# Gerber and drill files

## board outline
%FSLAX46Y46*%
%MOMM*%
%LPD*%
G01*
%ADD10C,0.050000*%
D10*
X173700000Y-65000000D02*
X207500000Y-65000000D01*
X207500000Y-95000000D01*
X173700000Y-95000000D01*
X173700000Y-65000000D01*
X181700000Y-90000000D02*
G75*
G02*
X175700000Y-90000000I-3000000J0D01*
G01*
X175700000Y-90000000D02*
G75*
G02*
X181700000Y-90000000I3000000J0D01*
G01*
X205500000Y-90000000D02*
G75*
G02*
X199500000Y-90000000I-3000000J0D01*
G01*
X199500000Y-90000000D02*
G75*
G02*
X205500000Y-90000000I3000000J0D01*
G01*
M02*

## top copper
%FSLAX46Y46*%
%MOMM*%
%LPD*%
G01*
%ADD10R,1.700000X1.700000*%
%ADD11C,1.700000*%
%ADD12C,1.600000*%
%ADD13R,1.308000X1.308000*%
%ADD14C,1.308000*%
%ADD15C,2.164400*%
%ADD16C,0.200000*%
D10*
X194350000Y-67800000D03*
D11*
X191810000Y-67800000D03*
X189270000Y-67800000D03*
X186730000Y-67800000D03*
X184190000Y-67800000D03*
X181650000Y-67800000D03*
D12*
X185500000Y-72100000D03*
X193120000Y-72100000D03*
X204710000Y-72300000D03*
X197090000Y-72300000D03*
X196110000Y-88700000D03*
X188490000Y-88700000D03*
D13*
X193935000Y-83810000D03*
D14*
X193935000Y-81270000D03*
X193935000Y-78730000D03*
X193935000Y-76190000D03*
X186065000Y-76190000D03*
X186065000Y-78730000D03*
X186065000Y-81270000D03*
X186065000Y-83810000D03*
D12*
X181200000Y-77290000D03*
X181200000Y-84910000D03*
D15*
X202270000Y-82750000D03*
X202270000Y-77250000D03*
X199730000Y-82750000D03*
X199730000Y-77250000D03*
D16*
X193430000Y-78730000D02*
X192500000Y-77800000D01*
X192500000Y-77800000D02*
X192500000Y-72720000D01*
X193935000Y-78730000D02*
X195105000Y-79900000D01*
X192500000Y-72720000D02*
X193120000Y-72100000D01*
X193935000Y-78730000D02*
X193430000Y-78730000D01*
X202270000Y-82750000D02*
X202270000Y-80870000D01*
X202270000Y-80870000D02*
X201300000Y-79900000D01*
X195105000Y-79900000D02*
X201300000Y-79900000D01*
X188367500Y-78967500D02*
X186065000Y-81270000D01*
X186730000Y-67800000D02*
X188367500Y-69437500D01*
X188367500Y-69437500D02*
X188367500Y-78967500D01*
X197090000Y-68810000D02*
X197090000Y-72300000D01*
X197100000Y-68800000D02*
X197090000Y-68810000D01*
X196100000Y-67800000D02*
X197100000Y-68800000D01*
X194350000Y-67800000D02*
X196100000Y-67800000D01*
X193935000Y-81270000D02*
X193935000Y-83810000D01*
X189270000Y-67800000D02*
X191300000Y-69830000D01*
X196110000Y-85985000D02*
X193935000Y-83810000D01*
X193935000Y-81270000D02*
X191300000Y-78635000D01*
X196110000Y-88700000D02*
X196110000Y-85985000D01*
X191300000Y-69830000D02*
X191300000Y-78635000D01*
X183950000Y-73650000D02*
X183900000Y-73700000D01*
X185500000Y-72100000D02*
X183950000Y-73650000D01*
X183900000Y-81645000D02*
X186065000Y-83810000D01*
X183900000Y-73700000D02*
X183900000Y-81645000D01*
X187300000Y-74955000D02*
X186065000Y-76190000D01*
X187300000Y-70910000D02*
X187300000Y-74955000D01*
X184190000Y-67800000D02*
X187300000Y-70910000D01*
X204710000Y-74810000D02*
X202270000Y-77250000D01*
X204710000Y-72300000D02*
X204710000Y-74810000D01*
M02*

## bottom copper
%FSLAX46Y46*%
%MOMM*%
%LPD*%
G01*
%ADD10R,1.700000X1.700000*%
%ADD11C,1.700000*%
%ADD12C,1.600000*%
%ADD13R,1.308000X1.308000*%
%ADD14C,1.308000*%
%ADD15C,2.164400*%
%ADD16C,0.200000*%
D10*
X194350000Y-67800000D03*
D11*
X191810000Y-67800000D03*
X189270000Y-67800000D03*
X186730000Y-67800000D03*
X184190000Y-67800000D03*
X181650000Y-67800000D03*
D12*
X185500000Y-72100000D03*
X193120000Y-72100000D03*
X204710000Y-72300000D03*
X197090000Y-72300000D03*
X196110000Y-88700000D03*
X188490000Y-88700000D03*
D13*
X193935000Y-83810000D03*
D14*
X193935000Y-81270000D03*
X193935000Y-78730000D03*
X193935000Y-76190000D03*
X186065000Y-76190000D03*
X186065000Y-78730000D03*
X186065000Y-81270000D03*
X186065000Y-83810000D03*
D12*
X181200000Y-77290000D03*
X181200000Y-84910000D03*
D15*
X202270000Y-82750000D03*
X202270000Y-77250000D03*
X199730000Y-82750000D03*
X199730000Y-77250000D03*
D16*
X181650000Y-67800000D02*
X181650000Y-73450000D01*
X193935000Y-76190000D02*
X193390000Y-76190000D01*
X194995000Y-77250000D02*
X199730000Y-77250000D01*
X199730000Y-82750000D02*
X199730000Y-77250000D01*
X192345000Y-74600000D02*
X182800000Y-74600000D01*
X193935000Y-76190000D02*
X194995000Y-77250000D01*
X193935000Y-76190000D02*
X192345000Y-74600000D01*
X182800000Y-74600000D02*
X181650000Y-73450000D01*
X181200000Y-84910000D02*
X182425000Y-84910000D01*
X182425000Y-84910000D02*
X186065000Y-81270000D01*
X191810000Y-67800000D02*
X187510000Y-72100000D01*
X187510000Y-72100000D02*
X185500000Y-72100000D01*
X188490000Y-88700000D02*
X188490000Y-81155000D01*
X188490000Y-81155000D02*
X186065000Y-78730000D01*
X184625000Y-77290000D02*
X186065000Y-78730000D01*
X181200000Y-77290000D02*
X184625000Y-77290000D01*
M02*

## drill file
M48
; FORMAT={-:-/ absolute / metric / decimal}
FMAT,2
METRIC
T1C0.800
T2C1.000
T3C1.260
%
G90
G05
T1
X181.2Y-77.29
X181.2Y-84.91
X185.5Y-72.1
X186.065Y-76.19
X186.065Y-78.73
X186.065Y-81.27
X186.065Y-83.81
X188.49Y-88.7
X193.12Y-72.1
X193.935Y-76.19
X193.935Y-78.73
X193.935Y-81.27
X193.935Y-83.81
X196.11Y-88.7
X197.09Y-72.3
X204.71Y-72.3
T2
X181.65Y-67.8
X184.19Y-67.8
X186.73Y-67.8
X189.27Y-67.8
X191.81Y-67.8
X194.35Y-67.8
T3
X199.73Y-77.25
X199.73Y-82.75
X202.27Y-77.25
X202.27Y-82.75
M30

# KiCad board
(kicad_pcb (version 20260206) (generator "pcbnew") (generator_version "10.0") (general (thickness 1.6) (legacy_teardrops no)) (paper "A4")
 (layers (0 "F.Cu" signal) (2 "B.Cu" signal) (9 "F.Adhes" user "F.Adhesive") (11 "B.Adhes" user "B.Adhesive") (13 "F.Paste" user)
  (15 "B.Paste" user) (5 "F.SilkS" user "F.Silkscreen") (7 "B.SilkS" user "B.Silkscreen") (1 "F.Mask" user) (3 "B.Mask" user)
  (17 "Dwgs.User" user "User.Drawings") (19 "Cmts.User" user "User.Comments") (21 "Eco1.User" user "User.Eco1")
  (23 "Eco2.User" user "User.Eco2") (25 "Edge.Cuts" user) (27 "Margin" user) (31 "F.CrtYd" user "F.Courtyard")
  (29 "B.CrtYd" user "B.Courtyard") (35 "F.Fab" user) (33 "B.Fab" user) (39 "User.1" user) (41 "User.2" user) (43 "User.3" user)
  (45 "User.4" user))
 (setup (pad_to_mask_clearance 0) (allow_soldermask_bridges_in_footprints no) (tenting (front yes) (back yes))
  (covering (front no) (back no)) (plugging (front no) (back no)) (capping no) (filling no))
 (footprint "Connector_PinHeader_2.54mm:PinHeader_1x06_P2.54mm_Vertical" (layer "F.Cu") (at 194.35 67.8 -90)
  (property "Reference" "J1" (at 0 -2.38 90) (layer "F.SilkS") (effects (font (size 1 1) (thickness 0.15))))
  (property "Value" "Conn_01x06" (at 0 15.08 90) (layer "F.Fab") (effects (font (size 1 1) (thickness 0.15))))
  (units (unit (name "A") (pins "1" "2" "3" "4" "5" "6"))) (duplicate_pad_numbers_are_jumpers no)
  (pad "1" thru_hole rect (at 0 0 270) (size 1.7 1.7) (drill 1) (layers "*.Cu" "*.Mask") (remove_unused_layers no) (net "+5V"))
  (pad "2" thru_hole circle (at 0 2.54 270) (size 1.7 1.7) (drill 1) (layers "*.Cu" "*.Mask") (remove_unused_layers no) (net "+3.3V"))
  (pad "3" thru_hole circle (at 0 5.08 270) (size 1.7 1.7) (drill 1) (layers "*.Cu" "*.Mask") (remove_unused_layers no) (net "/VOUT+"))
  (pad "4" thru_hole circle (at 0 7.62 270) (size 1.7 1.7) (drill 1) (layers "*.Cu" "*.Mask") (remove_unused_layers no) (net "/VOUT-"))
  (pad "5" thru_hole circle (at 0 10.16 270) (size 1.7 1.7) (drill 1) (layers "*.Cu" "*.Mask") (remove_unused_layers no) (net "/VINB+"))
  (pad "6" thru_hole circle (at 0 12.7 270) (size 1.7 1.7) (drill 1) (layers "*.Cu" "*.Mask") (remove_unused_layers no) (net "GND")))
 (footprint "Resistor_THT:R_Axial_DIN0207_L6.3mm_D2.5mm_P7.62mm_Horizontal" (layer "F.Cu") (at 185.5 72.1)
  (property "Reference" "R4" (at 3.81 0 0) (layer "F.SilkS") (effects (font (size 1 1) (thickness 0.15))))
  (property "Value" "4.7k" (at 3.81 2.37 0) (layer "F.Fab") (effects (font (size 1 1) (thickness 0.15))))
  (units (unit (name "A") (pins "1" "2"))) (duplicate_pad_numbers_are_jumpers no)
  (pad "1" thru_hole circle (at 0 0) (size 1.6 1.6) (drill 0.8) (layers "*.Cu" "*.Mask") (remove_unused_layers no) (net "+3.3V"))
  (pad "2" thru_hole circle (at 7.62 0) (size 1.6 1.6) (drill 0.8) (layers "*.Cu" "*.Mask") (remove_unused_layers no) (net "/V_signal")))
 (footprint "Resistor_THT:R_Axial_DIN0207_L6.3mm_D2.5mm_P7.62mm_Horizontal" (layer "F.Cu") (at 204.71 72.3 180)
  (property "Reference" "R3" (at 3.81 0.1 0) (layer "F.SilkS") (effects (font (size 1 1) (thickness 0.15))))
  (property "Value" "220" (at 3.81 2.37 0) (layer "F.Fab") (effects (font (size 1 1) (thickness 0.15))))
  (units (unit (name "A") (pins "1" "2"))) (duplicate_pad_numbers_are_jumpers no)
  (pad "1" thru_hole circle (at 0 0 180) (size 1.6 1.6) (drill 0.8) (layers "*.Cu" "*.Mask") (remove_unused_layers no) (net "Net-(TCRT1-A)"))
  (pad "2" thru_hole circle (at 7.62 0 180) (size 1.6 1.6) (drill 0.8) (layers "*.Cu" "*.Mask") (remove_unused_layers no) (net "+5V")))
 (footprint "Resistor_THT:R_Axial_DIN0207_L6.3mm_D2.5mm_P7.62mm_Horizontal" (layer "F.Cu") (at 196.11 88.7 180)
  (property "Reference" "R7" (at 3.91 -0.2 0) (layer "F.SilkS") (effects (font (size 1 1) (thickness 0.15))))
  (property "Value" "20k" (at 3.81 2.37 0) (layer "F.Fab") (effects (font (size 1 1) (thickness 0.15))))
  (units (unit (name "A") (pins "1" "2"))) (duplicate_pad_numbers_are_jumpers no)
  (pad "1" thru_hole circle (at 0 0 180) (size 1.6 1.6) (drill 0.8) (layers "*.Cu" "*.Mask") (remove_unused_layers no) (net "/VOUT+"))
  (pad "2" thru_hole circle (at 7.62 0 180) (size 1.6 1.6) (drill 0.8) (layers "*.Cu" "*.Mask") (remove_unused_layers no) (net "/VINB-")))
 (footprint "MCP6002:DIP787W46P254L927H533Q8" (layer "F.Cu") (at 190 80 180)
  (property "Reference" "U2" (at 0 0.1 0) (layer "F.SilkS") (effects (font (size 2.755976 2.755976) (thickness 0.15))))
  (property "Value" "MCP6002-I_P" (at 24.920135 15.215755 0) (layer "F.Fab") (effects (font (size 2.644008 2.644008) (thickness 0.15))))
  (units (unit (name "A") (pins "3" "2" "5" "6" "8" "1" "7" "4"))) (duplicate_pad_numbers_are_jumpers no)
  (pad "1" thru_hole rect (at -3.935 -3.81 180) (size 1.308 1.308) (drill 0.8) (layers "*.Cu" "*.Mask") (remove_unused_layers no)
   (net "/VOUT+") (solder_mask_margin 0.102))
  (pad "2" thru_hole circle (at -3.935 -1.27 180) (size 1.308 1.308) (drill 0.8) (layers "*.Cu" "*.Mask") (remove_unused_layers no)
   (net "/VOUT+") (solder_mask_margin 0.102))
  (pad "3" thru_hole circle (at -3.935 1.27 180) (size 1.308 1.308) (drill 0.8) (layers "*.Cu" "*.Mask") (remove_unused_layers no)
   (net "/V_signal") (solder_mask_margin 0.102))
  (pad "4" thru_hole circle (at -3.935 3.81 180) (size 1.308 1.308) (drill 0.8) (layers "*.Cu" "*.Mask") (remove_unused_layers no)
   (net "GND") (solder_mask_margin 0.102))
  (pad "5" thru_hole circle (at 3.935 3.81 180) (size 1.308 1.308) (drill 0.8) (layers "*.Cu" "*.Mask") (remove_unused_layers no)
   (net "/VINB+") (solder_mask_margin 0.102))
  (pad "6" thru_hole circle (at 3.935 1.27 180) (size 1.308 1.308) (drill 0.8) (layers "*.Cu" "*.Mask") (remove_unused_layers no)
   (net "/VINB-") (solder_mask_margin 0.102))
  (pad "7" thru_hole circle (at 3.935 -1.27 180) (size 1.308 1.308) (drill 0.8) (layers "*.Cu" "*.Mask") (remove_unused_layers no)
   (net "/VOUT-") (solder_mask_margin 0.102))
  (pad "8" thru_hole circle (at 3.935 -3.81 180) (size 1.308 1.308) (drill 0.8) (layers "*.Cu" "*.Mask") (remove_unused_layers no)
   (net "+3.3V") (solder_mask_margin 0.102)))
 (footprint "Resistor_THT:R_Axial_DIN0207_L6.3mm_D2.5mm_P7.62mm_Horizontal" (layer "F.Cu") (at 181.2 77.29 -90)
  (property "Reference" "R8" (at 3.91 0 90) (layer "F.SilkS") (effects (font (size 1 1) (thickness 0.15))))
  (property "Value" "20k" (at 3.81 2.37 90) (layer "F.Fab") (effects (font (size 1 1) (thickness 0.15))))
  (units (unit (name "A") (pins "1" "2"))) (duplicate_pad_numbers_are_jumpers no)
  (pad "1" thru_hole circle (at 0 0 270) (size 1.6 1.6) (drill 0.8) (layers "*.Cu" "*.Mask") (remove_unused_layers no) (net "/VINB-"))
  (pad "2" thru_hole circle (at 7.62 0 270) (size 1.6 1.6) (drill 0.8) (layers "*.Cu" "*.Mask") (remove_unused_layers no) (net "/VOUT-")))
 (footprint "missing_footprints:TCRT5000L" (layer "B.Cu") (at 201 80 90)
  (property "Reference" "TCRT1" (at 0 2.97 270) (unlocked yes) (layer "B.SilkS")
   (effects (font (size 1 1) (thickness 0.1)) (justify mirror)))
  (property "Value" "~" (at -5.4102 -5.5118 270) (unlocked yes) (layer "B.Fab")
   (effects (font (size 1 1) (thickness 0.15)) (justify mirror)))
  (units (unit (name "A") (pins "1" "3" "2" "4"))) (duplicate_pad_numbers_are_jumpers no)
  (pad "1" thru_hole circle (at -2.75 1.27 90) (size 2.1644 2.1644) (drill 1.26) (layers "*.Cu" "*.Mask") (remove_unused_layers no)
   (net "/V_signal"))
  (pad "2" thru_hole circle (at 2.75 1.27 90) (size 2.1644 2.1644) (drill 1.26) (layers "*.Cu" "*.Mask") (remove_unused_layers no)
   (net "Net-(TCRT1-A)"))
  (pad "3" thru_hole circle (at -2.75 -1.27 90) (size 2.1644 2.1644) (drill 1.26) (layers "*.Cu" "*.Mask") (remove_unused_layers no)
   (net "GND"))
  (pad "4" thru_hole circle (at 2.75 -1.27 90) (size 2.1644 2.1644) (drill 1.26) (layers "*.Cu" "*.Mask") (remove_unused_layers no)
   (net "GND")))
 (gr_rect (start 173.7 65) (end 207.5 95) (stroke (width 0.05) (type solid)) (fill no) (layer "Edge.Cuts"))
 (gr_circle (center 178.7 90) (end 181.7 90) (stroke (width 0.05) (type solid)) (fill no) (layer "Edge.Cuts"))
 (gr_circle (center 202.5 90) (end 205.5 90) (stroke (width 0.05) (type solid)) (fill no) (layer "Edge.Cuts"))
 (segment (start 181.65 67.8) (end 181.65 73.45) (width 0.2) (layer "B.Cu") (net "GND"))
 (segment (start 193.935 76.19) (end 193.39 76.19) (width 0.2) (layer "B.Cu") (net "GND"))
 (segment (start 194.995 77.25) (end 199.73 77.25) (width 0.2) (layer "B.Cu") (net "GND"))
 (segment (start 199.73 82.75) (end 199.73 77.25) (width 0.2) (layer "B.Cu") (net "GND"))
 (segment (start 192.345 74.6) (end 182.8 74.6) (width 0.2) (layer "B.Cu") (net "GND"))
 (segment (start 193.935 76.19) (end 194.995 77.25) (width 0.2) (layer "B.Cu") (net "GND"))
 (segment (start 193.935 76.19) (end 192.345 74.6) (width 0.2) (layer "B.Cu") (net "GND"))
 (segment (start 182.8 74.6) (end 181.65 73.45) (width 0.2) (layer "B.Cu") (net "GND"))
 (segment (start 193.43 78.73) (end 192.5 77.8) (width 0.2) (layer "F.Cu") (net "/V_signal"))
 (segment (start 192.5 77.8) (end 192.5 72.72) (width 0.2) (layer "F.Cu") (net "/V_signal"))
 (segment (start 193.935 78.73) (end 195.105 79.9) (width 0.2) (layer "F.Cu") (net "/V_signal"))
 (segment (start 192.5 72.72) (end 193.12 72.1) (width 0.2) (layer "F.Cu") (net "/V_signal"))
 (segment (start 193.935 78.73) (end 193.43 78.73) (width 0.2) (layer "F.Cu") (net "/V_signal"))
 (segment (start 202.27 82.75) (end 202.27 80.87) (width 0.2) (layer "F.Cu") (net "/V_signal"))
 (segment (start 202.27 80.87) (end 201.3 79.9) (width 0.2) (layer "F.Cu") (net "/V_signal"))
 (segment (start 195.105 79.9) (end 201.3 79.9) (width 0.2) (layer "F.Cu") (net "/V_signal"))
 (segment (start 188.3675 78.9675) (end 186.065 81.27) (width 0.2) (layer "F.Cu") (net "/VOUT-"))
 (segment (start 186.73 67.8) (end 188.3675 69.4375) (width 0.2) (layer "F.Cu") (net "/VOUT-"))
 (segment (start 188.3675 69.4375) (end 188.3675 78.9675) (width 0.2) (layer "F.Cu") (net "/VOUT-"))
 (segment (start 181.2 84.91) (end 182.425 84.91) (width 0.2) (layer "B.Cu") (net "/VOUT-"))
 (segment (start 182.425 84.91) (end 186.065 81.27) (width 0.2) (layer "B.Cu") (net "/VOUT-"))
 (segment (start 197.09 68.81) (end 197.09 72.3) (width 0.2) (layer "F.Cu") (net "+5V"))
 (segment (start 197.1 68.8) (end 197.09 68.81) (width 0.2) (layer "F.Cu") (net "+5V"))
 (segment (start 196.1 67.8) (end 197.1 68.8) (width 0.2) (layer "F.Cu") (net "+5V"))
 (segment (start 194.35 67.8) (end 196.1 67.8) (width 0.2) (layer "F.Cu") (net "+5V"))
 (segment (start 193.935 81.27) (end 193.935 83.81) (width 0.2) (layer "F.Cu") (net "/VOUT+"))
 (segment (start 189.27 67.8) (end 191.3 69.83) (width 0.2) (layer "F.Cu") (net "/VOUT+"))
 (segment (start 196.11 85.985) (end 193.935 83.81) (width 0.2) (layer "F.Cu") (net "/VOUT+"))
 (segment (start 193.935 81.27) (end 191.3 78.635) (width 0.2) (layer "F.Cu") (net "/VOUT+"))
 (segment (start 196.11 88.7) (end 196.11 85.985) (width 0.2) (layer "F.Cu") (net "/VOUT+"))
 (segment (start 191.3 69.83) (end 191.3 78.635) (width 0.2) (layer "F.Cu") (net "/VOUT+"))
 (segment (start 183.95 73.65) (end 183.9 73.7) (width 0.2) (layer "F.Cu") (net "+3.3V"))
 (segment (start 185.5 72.1) (end 183.95 73.65) (width 0.2) (layer "F.Cu") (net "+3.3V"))
 (segment (start 183.9 81.645) (end 186.065 83.81) (width 0.2) (layer "F.Cu") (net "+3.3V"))
 (segment (start 183.9 73.7) (end 183.9 81.645) (width 0.2) (layer "F.Cu") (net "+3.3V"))
 (segment (start 191.81 67.8) (end 187.51 72.1) (width 0.2) (layer "B.Cu") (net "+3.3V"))
 (segment (start 187.51 72.1) (end 185.5 72.1) (width 0.2) (layer "B.Cu") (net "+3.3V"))
 (segment (start 187.3 74.955) (end 186.065 76.19) (width 0.2) (layer "F.Cu") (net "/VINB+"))
 (segment (start 187.3 70.91) (end 187.3 74.955) (width 0.2) (layer "F.Cu") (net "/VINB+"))
 (segment (start 184.19 67.8) (end 187.3 70.91) (width 0.2) (layer "F.Cu") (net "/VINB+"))
 (segment (start 204.71 74.81) (end 202.27 77.25) (width 0.2) (layer "F.Cu") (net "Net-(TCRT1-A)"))
 (segment (start 204.71 72.3) (end 204.71 74.81) (width 0.2) (layer "F.Cu") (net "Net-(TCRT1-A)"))
 (segment (start 188.49 88.7) (end 188.49 81.155) (width 0.2) (layer "B.Cu") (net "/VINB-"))
 (segment (start 188.49 81.155) (end 186.065 78.73) (width 0.2) (layer "B.Cu") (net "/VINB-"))
 (segment (start 184.625 77.29) (end 186.065 78.73) (width 0.2) (layer "B.Cu") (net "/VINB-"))
 (segment (start 181.2 77.29) (end 184.625 77.29) (width 0.2) (layer "B.Cu") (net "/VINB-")))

